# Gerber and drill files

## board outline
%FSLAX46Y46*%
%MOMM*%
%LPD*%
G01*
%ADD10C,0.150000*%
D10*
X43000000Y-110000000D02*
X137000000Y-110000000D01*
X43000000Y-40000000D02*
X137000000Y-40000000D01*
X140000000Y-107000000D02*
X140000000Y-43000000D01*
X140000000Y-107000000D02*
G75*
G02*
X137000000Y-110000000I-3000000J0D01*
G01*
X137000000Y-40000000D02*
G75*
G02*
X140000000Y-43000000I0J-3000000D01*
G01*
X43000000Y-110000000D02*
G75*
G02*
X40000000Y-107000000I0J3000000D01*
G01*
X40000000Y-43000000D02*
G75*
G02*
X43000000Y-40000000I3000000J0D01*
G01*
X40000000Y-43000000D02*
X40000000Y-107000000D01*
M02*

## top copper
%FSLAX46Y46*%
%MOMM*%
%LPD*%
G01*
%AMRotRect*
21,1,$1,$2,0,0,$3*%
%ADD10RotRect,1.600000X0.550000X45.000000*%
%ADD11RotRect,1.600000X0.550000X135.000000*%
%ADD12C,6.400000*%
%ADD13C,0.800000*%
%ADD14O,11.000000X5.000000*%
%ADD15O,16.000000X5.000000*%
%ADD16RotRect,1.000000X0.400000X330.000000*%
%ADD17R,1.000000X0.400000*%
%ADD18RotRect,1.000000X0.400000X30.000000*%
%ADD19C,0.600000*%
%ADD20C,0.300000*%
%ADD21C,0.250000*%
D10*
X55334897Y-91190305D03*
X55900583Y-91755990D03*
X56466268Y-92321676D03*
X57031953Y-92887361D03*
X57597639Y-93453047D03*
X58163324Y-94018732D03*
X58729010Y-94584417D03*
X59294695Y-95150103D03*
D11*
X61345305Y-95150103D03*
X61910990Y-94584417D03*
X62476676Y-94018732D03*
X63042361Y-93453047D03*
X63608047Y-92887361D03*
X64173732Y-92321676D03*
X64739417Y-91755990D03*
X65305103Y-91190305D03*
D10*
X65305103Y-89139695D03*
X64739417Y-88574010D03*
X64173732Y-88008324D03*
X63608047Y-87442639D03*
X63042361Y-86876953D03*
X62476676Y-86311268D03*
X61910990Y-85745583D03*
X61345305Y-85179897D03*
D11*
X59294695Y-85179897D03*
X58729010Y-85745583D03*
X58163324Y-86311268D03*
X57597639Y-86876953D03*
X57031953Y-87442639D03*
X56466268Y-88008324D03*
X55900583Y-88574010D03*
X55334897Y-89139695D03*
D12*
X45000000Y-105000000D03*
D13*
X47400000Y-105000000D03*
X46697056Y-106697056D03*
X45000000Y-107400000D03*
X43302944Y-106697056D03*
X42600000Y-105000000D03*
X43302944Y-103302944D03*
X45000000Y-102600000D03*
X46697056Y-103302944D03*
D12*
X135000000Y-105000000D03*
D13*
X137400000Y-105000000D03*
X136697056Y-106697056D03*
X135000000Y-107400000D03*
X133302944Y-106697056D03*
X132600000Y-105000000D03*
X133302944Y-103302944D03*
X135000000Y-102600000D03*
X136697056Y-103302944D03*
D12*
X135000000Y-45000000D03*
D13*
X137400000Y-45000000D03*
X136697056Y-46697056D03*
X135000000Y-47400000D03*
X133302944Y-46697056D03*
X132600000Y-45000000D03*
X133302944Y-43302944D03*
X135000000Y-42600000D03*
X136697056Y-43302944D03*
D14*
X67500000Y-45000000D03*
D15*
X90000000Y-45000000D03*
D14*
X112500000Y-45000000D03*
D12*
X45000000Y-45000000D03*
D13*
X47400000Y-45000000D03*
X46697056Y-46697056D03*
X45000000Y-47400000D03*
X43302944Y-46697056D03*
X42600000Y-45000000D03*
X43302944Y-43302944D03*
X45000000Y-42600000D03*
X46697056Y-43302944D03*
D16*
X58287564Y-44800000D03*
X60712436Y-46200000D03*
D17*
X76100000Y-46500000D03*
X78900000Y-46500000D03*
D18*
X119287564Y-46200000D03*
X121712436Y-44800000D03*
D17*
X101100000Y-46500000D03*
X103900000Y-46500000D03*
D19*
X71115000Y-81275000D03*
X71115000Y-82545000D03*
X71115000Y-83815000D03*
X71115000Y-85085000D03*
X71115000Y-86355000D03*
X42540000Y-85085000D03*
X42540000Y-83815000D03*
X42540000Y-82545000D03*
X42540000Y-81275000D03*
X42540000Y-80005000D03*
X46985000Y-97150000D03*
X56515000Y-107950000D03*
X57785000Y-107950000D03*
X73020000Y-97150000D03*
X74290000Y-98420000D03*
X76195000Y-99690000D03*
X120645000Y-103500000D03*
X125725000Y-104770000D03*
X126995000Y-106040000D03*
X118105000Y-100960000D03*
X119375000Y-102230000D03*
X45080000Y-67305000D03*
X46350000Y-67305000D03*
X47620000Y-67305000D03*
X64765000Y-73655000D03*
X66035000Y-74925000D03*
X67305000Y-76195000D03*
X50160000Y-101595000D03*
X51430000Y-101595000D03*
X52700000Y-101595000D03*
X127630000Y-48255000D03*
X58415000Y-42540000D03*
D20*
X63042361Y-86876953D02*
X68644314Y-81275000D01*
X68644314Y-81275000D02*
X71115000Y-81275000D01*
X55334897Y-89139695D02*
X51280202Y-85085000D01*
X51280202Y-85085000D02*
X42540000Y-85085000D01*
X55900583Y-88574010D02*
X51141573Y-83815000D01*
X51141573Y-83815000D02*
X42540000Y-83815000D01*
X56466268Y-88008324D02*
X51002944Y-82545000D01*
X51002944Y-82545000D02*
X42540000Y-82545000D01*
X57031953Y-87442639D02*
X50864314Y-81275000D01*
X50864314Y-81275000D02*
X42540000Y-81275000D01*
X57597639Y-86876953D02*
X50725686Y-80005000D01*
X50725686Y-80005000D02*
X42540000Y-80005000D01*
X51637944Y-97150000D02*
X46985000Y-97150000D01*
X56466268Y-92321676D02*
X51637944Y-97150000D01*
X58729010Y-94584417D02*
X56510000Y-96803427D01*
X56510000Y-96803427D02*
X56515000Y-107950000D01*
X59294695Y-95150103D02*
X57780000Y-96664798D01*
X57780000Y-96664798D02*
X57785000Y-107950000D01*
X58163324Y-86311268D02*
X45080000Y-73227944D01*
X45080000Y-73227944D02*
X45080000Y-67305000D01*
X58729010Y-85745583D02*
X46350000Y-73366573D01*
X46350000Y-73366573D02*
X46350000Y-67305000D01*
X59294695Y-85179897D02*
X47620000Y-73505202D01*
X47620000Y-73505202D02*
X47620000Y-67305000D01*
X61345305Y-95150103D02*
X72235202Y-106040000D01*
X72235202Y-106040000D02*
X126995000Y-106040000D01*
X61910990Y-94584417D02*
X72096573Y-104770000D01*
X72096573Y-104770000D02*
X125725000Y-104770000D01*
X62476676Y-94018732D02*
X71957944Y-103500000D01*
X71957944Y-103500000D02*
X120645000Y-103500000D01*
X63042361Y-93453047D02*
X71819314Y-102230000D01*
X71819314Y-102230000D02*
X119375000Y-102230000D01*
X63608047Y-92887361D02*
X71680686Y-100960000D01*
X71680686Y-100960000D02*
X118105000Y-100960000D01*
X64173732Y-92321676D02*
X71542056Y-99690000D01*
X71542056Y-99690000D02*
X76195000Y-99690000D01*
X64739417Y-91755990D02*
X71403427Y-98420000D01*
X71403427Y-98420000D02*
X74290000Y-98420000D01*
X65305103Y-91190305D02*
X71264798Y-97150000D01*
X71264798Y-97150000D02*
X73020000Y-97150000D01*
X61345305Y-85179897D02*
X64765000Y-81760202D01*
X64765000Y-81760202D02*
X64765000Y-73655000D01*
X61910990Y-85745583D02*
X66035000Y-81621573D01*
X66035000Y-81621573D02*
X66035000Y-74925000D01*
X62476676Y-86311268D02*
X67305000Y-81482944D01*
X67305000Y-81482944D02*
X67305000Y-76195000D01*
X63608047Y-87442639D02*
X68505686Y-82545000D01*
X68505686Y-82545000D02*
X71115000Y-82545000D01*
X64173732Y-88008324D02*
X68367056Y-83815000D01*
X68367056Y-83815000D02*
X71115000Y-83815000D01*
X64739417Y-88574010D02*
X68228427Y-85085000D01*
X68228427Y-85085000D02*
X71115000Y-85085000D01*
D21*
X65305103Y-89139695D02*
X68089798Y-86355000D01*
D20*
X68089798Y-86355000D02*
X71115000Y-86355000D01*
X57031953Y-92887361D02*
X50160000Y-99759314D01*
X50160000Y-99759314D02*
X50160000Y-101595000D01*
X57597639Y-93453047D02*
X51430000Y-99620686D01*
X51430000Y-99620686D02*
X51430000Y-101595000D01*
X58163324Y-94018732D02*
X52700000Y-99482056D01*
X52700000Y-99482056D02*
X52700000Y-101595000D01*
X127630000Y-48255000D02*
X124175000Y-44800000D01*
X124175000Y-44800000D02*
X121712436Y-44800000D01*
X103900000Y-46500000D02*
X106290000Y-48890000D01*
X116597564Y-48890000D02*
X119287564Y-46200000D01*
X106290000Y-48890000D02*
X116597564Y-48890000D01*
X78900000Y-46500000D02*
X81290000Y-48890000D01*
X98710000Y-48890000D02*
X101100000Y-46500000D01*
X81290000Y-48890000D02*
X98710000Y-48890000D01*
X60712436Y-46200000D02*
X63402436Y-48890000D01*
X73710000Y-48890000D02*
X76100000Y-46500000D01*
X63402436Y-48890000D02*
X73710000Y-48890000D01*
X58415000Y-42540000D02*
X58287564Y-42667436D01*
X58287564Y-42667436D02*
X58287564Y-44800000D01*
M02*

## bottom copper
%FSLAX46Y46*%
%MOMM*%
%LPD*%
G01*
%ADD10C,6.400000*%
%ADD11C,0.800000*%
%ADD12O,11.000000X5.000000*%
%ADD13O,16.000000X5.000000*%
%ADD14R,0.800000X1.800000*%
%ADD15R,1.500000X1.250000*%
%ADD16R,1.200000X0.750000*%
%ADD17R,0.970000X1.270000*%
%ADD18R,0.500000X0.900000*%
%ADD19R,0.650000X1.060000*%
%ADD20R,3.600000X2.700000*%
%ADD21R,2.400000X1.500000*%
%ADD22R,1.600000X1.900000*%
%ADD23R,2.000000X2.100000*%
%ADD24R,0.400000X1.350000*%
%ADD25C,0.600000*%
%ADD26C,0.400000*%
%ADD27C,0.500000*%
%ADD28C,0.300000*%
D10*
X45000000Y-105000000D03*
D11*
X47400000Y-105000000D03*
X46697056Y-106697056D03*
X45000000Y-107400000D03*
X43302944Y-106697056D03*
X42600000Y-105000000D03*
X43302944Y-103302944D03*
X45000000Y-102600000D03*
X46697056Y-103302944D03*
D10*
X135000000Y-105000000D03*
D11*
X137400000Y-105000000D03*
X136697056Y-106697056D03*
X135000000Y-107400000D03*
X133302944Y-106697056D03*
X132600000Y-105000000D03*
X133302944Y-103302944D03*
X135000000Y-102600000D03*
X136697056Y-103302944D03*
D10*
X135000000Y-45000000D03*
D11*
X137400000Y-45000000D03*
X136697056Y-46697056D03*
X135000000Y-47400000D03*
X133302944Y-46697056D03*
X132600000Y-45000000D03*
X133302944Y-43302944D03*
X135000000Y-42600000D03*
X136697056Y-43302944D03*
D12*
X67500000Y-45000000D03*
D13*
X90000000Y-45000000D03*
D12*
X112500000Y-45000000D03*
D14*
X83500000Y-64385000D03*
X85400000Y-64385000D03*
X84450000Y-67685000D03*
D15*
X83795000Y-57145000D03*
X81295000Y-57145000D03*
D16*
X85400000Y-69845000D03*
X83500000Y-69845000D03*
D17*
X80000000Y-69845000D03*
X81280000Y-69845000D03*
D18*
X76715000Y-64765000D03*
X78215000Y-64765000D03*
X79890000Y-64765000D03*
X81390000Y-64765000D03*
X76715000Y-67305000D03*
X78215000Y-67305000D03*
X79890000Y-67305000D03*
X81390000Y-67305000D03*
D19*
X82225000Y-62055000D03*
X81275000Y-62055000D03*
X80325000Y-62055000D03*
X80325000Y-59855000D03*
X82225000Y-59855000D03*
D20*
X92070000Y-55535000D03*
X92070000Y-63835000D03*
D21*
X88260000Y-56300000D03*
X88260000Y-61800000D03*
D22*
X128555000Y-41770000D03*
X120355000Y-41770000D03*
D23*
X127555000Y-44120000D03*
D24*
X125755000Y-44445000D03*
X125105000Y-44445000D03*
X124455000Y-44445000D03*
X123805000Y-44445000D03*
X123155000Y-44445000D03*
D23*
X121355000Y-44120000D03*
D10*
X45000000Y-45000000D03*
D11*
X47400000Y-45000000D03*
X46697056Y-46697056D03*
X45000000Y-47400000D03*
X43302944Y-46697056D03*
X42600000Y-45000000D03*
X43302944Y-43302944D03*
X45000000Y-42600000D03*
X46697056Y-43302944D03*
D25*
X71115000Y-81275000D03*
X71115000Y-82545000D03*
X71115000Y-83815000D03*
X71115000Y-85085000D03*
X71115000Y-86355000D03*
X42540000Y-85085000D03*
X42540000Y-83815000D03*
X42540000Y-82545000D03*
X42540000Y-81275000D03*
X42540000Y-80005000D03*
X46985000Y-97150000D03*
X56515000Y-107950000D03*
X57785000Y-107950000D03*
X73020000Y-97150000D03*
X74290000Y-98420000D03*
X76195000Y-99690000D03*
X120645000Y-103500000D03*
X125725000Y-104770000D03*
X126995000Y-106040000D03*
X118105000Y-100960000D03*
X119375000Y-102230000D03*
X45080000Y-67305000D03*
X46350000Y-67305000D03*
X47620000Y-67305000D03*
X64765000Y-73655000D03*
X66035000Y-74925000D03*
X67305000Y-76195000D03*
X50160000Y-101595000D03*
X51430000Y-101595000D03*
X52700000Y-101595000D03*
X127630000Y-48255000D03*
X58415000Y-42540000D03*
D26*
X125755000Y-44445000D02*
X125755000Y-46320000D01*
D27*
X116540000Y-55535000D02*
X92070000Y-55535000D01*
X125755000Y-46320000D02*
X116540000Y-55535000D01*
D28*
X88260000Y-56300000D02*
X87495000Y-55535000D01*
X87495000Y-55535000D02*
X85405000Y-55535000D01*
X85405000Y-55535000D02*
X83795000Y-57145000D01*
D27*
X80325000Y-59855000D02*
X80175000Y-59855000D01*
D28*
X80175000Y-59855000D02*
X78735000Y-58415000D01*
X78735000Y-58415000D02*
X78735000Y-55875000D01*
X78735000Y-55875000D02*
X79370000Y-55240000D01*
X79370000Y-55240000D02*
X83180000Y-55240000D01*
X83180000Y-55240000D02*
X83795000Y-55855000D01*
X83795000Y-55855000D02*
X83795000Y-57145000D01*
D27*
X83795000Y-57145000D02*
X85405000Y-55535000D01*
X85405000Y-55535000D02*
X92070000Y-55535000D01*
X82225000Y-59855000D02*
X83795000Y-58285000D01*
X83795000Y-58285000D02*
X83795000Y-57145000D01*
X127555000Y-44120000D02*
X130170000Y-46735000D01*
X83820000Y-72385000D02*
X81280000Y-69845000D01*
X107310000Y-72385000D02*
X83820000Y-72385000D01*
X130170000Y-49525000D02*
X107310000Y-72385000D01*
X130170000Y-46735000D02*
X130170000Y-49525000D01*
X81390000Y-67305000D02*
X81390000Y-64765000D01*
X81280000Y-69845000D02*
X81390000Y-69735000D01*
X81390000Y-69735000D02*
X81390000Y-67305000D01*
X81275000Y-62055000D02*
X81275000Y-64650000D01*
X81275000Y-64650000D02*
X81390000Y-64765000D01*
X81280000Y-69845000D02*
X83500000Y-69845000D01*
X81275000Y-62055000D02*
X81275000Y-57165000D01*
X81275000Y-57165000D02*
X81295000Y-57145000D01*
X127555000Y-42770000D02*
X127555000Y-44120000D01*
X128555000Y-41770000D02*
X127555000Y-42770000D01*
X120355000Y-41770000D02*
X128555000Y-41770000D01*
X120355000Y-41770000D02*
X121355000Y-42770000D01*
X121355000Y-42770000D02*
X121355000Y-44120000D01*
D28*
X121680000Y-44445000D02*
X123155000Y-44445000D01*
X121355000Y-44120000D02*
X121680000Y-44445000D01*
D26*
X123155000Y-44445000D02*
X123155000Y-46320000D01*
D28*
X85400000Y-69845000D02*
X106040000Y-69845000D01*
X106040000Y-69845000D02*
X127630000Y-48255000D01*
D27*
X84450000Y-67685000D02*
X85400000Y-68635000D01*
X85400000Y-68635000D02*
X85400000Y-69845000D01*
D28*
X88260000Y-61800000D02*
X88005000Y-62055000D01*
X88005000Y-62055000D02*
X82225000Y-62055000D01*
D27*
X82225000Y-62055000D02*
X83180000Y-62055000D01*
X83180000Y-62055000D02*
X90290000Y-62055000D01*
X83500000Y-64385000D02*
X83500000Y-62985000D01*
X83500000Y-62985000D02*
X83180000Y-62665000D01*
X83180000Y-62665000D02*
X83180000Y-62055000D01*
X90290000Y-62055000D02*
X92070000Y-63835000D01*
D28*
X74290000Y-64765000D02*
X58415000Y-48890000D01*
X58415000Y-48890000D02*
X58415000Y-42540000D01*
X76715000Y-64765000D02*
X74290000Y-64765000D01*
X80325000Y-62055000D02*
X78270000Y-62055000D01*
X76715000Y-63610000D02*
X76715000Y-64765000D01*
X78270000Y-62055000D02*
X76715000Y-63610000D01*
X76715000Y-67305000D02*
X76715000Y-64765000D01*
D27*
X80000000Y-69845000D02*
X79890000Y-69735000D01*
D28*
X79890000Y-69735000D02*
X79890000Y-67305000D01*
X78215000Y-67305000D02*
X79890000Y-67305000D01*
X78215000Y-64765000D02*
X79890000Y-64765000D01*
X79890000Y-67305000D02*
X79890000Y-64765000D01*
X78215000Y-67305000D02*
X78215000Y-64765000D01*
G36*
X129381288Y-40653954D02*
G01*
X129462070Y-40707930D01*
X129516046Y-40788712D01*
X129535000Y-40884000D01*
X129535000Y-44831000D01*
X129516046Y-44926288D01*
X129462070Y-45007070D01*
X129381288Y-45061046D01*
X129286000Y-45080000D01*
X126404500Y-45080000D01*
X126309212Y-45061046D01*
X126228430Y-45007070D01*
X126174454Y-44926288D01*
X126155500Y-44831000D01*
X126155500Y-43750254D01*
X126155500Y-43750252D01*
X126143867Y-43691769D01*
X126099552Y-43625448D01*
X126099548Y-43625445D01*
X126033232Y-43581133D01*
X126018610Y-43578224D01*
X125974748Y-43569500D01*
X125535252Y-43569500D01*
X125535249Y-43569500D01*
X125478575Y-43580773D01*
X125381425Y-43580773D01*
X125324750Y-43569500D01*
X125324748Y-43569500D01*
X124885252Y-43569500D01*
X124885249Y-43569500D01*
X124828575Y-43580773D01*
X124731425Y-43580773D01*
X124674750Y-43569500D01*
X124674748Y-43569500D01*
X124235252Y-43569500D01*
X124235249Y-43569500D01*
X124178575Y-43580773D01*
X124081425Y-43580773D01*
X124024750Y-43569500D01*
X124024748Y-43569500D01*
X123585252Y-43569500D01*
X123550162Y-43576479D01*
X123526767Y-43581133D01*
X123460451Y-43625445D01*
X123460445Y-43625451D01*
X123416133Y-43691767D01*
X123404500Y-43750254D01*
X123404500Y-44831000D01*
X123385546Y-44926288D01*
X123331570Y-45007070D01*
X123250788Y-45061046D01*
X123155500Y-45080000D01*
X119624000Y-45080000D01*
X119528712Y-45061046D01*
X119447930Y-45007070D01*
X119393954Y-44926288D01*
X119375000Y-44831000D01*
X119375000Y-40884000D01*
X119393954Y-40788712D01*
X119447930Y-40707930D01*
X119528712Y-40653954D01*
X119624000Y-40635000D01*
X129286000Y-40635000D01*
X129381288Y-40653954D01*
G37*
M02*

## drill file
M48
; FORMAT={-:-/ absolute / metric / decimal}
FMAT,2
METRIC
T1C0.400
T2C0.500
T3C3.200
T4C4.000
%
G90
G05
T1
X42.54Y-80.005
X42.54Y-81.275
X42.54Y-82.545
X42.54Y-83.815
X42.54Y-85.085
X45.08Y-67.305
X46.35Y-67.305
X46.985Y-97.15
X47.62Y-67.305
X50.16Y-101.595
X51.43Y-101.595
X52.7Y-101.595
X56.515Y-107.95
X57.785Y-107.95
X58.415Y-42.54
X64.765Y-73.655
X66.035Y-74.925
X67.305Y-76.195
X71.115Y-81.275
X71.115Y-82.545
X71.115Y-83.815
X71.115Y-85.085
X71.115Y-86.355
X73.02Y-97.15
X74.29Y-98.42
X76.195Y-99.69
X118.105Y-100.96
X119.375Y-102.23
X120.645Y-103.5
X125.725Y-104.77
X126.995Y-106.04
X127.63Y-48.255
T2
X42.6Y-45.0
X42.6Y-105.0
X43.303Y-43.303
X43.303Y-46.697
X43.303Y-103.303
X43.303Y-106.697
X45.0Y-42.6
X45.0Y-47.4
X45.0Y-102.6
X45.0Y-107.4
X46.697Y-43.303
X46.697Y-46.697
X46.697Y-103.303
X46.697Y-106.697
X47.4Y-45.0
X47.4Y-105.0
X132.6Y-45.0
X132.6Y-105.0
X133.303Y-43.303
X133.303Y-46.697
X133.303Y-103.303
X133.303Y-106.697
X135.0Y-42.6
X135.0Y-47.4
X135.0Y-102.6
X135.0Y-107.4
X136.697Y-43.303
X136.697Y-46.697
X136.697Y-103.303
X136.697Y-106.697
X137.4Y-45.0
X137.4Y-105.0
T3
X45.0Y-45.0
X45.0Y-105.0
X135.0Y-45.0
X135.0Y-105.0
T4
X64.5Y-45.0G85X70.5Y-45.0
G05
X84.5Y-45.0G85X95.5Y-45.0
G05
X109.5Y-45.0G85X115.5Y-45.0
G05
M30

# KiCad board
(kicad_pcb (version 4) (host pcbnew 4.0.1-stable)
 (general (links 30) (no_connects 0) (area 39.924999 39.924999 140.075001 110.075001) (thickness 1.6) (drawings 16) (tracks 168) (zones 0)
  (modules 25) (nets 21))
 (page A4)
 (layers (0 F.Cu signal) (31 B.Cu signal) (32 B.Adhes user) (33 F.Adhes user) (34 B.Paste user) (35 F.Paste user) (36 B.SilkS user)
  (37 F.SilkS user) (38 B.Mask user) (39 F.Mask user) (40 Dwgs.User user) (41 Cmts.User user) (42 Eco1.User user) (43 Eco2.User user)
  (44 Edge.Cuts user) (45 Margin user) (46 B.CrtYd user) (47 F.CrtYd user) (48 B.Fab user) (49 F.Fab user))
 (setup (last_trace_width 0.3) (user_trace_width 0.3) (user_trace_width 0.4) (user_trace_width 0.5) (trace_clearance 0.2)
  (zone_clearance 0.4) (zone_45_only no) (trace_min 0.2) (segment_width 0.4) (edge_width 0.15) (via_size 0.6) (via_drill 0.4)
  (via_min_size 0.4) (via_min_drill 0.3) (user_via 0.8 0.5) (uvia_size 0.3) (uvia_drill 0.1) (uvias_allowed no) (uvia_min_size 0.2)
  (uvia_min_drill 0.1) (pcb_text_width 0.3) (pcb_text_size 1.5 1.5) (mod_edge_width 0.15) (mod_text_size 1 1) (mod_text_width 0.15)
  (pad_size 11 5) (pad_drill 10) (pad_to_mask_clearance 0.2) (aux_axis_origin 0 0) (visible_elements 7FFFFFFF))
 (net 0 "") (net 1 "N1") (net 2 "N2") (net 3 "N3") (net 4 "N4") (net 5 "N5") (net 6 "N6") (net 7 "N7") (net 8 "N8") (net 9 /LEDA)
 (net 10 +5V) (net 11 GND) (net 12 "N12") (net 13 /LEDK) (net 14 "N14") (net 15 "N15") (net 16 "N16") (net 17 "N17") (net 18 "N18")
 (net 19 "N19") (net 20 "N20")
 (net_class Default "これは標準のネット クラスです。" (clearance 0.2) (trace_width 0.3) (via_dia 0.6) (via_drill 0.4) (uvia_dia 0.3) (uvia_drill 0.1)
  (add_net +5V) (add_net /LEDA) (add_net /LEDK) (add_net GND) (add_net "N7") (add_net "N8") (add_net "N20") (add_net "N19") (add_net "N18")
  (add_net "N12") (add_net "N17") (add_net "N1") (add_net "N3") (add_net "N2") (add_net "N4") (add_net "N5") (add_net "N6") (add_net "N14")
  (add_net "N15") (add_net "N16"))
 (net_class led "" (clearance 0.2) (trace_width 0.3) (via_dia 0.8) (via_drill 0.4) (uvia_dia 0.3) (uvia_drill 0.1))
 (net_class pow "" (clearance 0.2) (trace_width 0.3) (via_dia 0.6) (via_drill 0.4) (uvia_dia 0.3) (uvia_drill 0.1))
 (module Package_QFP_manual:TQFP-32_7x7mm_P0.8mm (layer F.Cu) (at 60.32 90.165 45)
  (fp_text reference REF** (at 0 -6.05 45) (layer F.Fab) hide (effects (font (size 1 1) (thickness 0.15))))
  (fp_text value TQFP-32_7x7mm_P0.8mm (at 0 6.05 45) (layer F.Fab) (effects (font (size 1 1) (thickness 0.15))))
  (pad 1 smd rect (at -4.25 -2.8 45) (size 1.6 0.55) (layers F.Cu F.Paste F.Mask))
  (pad 2 smd rect (at -4.25 -2 45) (size 1.6 0.55) (layers F.Cu F.Paste F.Mask))
  (pad 3 smd rect (at -4.25 -1.2 45) (size 1.6 0.55) (layers F.Cu F.Paste F.Mask))
  (pad 4 smd rect (at -4.25 -0.4 45) (size 1.6 0.55) (layers F.Cu F.Paste F.Mask))
  (pad 5 smd rect (at -4.25 0.4 45) (size 1.6 0.55) (layers F.Cu F.Paste F.Mask))
  (pad 6 smd rect (at -4.25 1.2 45) (size 1.6 0.55) (layers F.Cu F.Paste F.Mask))
  (pad 7 smd rect (at -4.25 2 45) (size 1.6 0.55) (layers F.Cu F.Paste F.Mask))
  (pad 8 smd rect (at -4.25 2.8 45) (size 1.6 0.55) (layers F.Cu F.Paste F.Mask))
  (pad 9 smd rect (at -2.8 4.25 135) (size 1.6 0.55) (layers F.Cu F.Paste F.Mask))
  (pad 10 smd rect (at -2 4.25 135) (size 1.6 0.55) (layers F.Cu F.Paste F.Mask))
  (pad 11 smd rect (at -1.2 4.25 135) (size 1.6 0.55) (layers F.Cu F.Paste F.Mask))
  (pad 12 smd rect (at -0.4 4.25 135) (size 1.6 0.55) (layers F.Cu F.Paste F.Mask))
  (pad 13 smd rect (at 0.4 4.25 135) (size 1.6 0.55) (layers F.Cu F.Paste F.Mask))
  (pad 14 smd rect (at 1.2 4.25 135) (size 1.6 0.55) (layers F.Cu F.Paste F.Mask))
  (pad 15 smd rect (at 2 4.25 135) (size 1.6 0.55) (layers F.Cu F.Paste F.Mask))
  (pad 16 smd rect (at 2.8 4.25 135) (size 1.6 0.55) (layers F.Cu F.Paste F.Mask))
  (pad 17 smd rect (at 4.25 2.8 45) (size 1.6 0.55) (layers F.Cu F.Paste F.Mask))
  (pad 18 smd rect (at 4.25 2 45) (size 1.6 0.55) (layers F.Cu F.Paste F.Mask))
  (pad 19 smd rect (at 4.25 1.2 45) (size 1.6 0.55) (layers F.Cu F.Paste F.Mask))
  (pad 20 smd rect (at 4.25 0.4 45) (size 1.6 0.55) (layers F.Cu F.Paste F.Mask))
  (pad 21 smd rect (at 4.25 -0.4 45) (size 1.6 0.55) (layers F.Cu F.Paste F.Mask))
  (pad 22 smd rect (at 4.25 -1.2 45) (size 1.6 0.55) (layers F.Cu F.Paste F.Mask))
  (pad 23 smd rect (at 4.25 -2 45) (size 1.6 0.55) (layers F.Cu F.Paste F.Mask))
  (pad 24 smd rect (at 4.25 -2.8 45) (size 1.6 0.55) (layers F.Cu F.Paste F.Mask))
  (pad 25 smd rect (at 2.8 -4.25 135) (size 1.6 0.55) (layers F.Cu F.Paste F.Mask))
  (pad 26 smd rect (at 2 -4.25 135) (size 1.6 0.55) (layers F.Cu F.Paste F.Mask))
  (pad 27 smd rect (at 1.2 -4.25 135) (size 1.6 0.55) (layers F.Cu F.Paste F.Mask))
  (pad 28 smd rect (at 0.4 -4.25 135) (size 1.6 0.55) (layers F.Cu F.Paste F.Mask))
  (pad 29 smd rect (at -0.4 -4.25 135) (size 1.6 0.55) (layers F.Cu F.Paste F.Mask))
  (pad 30 smd rect (at -1.2 -4.25 135) (size 1.6 0.55) (layers F.Cu F.Paste F.Mask))
  (pad 31 smd rect (at -2 -4.25 135) (size 1.6 0.55) (layers F.Cu F.Paste F.Mask))
  (pad 32 smd rect (at -2.8 -4.25 135) (size 1.6 0.55) (layers F.Cu F.Paste F.Mask)))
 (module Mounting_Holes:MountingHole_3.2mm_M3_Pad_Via (layer F.Cu) (at 45 105)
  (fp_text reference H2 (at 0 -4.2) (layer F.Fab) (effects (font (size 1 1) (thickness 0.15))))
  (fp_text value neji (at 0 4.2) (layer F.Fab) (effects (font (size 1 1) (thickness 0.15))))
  (pad 1 thru_hole circle (at 0 0) (size 6.4 6.4) (drill 3.2) (layers *.Cu *.Mask) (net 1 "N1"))
  (pad "" thru_hole circle (at 2.4 0) (size 0.8 0.8) (drill 0.5) (layers *.Cu *.Mask))
  (pad "" thru_hole circle (at 1.697056 1.697056) (size 0.8 0.8) (drill 0.5) (layers *.Cu *.Mask))
  (pad "" thru_hole circle (at 0 2.4) (size 0.8 0.8) (drill 0.5) (layers *.Cu *.Mask))
  (pad "" thru_hole circle (at -1.697056 1.697056) (size 0.8 0.8) (drill 0.5) (layers *.Cu *.Mask))
  (pad "" thru_hole circle (at -2.4 0) (size 0.8 0.8) (drill 0.5) (layers *.Cu *.Mask))
  (pad "" thru_hole circle (at -1.697056 -1.697056) (size 0.8 0.8) (drill 0.5) (layers *.Cu *.Mask))
  (pad "" thru_hole circle (at 0 -2.4) (size 0.8 0.8) (drill 0.5) (layers *.Cu *.Mask))
  (pad "" thru_hole circle (at 1.697056 -1.697056) (size 0.8 0.8) (drill 0.5) (layers *.Cu *.Mask)))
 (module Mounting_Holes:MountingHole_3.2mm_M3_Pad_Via (layer F.Cu) (at 135 105)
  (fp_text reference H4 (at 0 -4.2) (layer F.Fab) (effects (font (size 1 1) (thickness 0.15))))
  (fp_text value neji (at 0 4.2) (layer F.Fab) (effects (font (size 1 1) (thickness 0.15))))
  (pad 1 thru_hole circle (at 0 0) (size 6.4 6.4) (drill 3.2) (layers *.Cu *.Mask) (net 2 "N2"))
  (pad "" thru_hole circle (at 2.4 0) (size 0.8 0.8) (drill 0.5) (layers *.Cu *.Mask))
  (pad "" thru_hole circle (at 1.697056 1.697056) (size 0.8 0.8) (drill 0.5) (layers *.Cu *.Mask))
  (pad "" thru_hole circle (at 0 2.4) (size 0.8 0.8) (drill 0.5) (layers *.Cu *.Mask))
  (pad "" thru_hole circle (at -1.697056 1.697056) (size 0.8 0.8) (drill 0.5) (layers *.Cu *.Mask))
  (pad "" thru_hole circle (at -2.4 0) (size 0.8 0.8) (drill 0.5) (layers *.Cu *.Mask))
  (pad "" thru_hole circle (at -1.697056 -1.697056) (size 0.8 0.8) (drill 0.5) (layers *.Cu *.Mask))
  (pad "" thru_hole circle (at 0 -2.4) (size 0.8 0.8) (drill 0.5) (layers *.Cu *.Mask))
  (pad "" thru_hole circle (at 1.697056 -1.697056) (size 0.8 0.8) (drill 0.5) (layers *.Cu *.Mask)))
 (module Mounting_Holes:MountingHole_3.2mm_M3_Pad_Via (layer F.Cu) (at 135 45)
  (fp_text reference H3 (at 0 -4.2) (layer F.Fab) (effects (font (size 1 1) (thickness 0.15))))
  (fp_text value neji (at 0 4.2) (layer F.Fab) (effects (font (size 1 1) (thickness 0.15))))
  (pad 1 thru_hole circle (at 0 0) (size 6.4 6.4) (drill 3.2) (layers *.Cu *.Mask) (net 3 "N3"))
  (pad "" thru_hole circle (at 2.4 0) (size 0.8 0.8) (drill 0.5) (layers *.Cu *.Mask))
  (pad "" thru_hole circle (at 1.697056 1.697056) (size 0.8 0.8) (drill 0.5) (layers *.Cu *.Mask))
  (pad "" thru_hole circle (at 0 2.4) (size 0.8 0.8) (drill 0.5) (layers *.Cu *.Mask))
  (pad "" thru_hole circle (at -1.697056 1.697056) (size 0.8 0.8) (drill 0.5) (layers *.Cu *.Mask))
  (pad "" thru_hole circle (at -2.4 0) (size 0.8 0.8) (drill 0.5) (layers *.Cu *.Mask))
  (pad "" thru_hole circle (at -1.697056 -1.697056) (size 0.8 0.8) (drill 0.5) (layers *.Cu *.Mask))
  (pad "" thru_hole circle (at 0 -2.4) (size 0.8 0.8) (drill 0.5) (layers *.Cu *.Mask))
  (pad "" thru_hole circle (at 1.697056 -1.697056) (size 0.8 0.8) (drill 0.5) (layers *.Cu *.Mask)))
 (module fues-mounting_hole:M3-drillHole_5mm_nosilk (layer F.Cu) (at 67.5 45)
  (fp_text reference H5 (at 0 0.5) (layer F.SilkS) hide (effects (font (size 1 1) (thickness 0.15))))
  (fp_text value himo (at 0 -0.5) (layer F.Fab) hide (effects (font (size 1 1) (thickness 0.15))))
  (pad 1 thru_hole oval (at 0 0) (size 11 5) (drill oval 10 4) (layers *.Cu *.Mask) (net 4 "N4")))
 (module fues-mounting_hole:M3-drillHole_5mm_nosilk (layer F.Cu) (at 90 45)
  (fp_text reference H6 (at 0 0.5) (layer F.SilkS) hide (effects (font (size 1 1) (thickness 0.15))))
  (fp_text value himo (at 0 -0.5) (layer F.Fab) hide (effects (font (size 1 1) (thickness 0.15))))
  (pad 1 thru_hole oval (at 0 0) (size 16 5) (drill oval 15 4) (layers *.Cu *.Mask) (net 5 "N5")))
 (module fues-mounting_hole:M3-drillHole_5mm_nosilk (layer F.Cu) (at 112.5 45)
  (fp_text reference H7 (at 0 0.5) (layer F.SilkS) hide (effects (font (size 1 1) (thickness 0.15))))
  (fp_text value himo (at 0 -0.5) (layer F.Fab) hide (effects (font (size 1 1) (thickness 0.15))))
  (pad 1 thru_hole oval (at 0 0) (size 11 5) (drill oval 10 4) (layers *.Cu *.Mask) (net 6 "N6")))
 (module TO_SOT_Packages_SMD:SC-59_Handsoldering (layer B.Cu) (at 84.45 66.035 270)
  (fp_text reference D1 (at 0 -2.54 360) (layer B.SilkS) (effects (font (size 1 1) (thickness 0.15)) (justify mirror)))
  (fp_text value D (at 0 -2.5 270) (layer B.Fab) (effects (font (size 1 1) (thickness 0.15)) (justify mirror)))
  (pad 1 smd rect (at -1.65 0.95 270) (size 1.8 0.8) (layers B.Cu B.Paste B.Mask) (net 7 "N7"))
  (pad 2 smd rect (at -1.65 -0.95 270) (size 1.8 0.8) (layers B.Cu B.Paste B.Mask) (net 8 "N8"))
  (pad 3 smd rect (at 1.65 0 270) (size 1.8 0.8) (layers B.Cu B.Paste B.Mask) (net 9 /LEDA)))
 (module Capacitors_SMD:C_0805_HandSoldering (layer B.Cu) (at 82.545 57.145 180)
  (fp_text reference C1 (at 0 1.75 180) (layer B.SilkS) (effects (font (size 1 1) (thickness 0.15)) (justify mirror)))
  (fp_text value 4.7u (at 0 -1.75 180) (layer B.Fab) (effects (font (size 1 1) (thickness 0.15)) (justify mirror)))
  (pad 1 smd rect (at -1.25 0 180) (size 1.5 1.25) (layers B.Cu B.Paste B.Mask) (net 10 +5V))
  (pad 2 smd rect (at 1.25 0 180) (size 1.5 1.25) (layers B.Cu B.Paste B.Mask) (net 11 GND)))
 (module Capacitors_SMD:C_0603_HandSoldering (layer B.Cu) (at 84.45 69.845 180)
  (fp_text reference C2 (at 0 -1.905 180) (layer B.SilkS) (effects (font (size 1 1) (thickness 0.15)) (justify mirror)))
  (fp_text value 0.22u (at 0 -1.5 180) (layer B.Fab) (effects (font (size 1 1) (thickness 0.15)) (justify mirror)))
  (pad 1 smd rect (at -0.95 0 180) (size 1.2 0.75) (layers B.Cu B.Paste B.Mask) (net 9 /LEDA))
  (pad 2 smd rect (at 0.95 0 180) (size 1.2 0.75) (layers B.Cu B.Paste B.Mask) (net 11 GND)))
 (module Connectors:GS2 (layer B.Cu) (at 80.64 69.845 270)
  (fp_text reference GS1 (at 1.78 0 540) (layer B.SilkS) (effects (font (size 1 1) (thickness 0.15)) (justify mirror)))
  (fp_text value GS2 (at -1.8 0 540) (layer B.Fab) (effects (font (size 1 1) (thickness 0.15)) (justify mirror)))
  (pad 1 smd rect (at 0 0.64 270) (size 1.27 0.97) (layers B.Cu B.Paste B.Mask) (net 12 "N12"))
  (pad 2 smd rect (at 0 -0.64 270) (size 1.27 0.97) (layers B.Cu B.Paste B.Mask) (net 11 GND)))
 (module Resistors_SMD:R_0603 (layer B.Cu) (at 77.465 64.765)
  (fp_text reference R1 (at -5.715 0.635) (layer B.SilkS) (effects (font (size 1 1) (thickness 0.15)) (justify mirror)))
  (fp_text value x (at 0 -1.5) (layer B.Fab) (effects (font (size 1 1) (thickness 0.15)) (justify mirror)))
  (pad 1 smd rect (at -0.75 0) (size 0.5 0.9) (layers B.Cu B.Paste B.Mask) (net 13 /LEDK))
  (pad 2 smd rect (at 0.75 0) (size 0.5 0.9) (layers B.Cu B.Paste B.Mask) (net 12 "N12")))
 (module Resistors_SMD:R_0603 (layer B.Cu) (at 80.64 64.765)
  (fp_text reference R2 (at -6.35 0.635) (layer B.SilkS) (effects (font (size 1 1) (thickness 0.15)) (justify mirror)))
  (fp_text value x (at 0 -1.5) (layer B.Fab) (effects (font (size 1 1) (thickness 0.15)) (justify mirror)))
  (pad 1 smd rect (at -0.75 0) (size 0.5 0.9) (layers B.Cu B.Paste B.Mask) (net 12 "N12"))
  (pad 2 smd rect (at 0.75 0) (size 0.5 0.9) (layers B.Cu B.Paste B.Mask) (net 11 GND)))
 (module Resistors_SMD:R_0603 (layer B.Cu) (at 77.465 67.305)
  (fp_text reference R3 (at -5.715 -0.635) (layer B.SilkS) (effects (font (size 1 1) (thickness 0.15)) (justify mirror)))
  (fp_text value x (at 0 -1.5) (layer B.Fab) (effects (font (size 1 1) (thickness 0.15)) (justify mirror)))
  (pad 1 smd rect (at -0.75 0) (size 0.5 0.9) (layers B.Cu B.Paste B.Mask) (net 13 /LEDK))
  (pad 2 smd rect (at 0.75 0) (size 0.5 0.9) (layers B.Cu B.Paste B.Mask) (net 12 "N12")))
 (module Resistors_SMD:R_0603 (layer B.Cu) (at 80.64 67.305)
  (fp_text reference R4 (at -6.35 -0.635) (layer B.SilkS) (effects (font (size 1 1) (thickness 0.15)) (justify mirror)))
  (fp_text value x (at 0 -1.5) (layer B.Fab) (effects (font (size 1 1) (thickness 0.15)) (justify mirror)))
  (pad 1 smd rect (at -0.75 0) (size 0.5 0.9) (layers B.Cu B.Paste B.Mask) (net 12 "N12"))
  (pad 2 smd rect (at 0.75 0) (size 0.5 0.9) (layers B.Cu B.Paste B.Mask) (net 11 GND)))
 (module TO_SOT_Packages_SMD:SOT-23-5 (layer B.Cu) (at 81.275 60.955 90)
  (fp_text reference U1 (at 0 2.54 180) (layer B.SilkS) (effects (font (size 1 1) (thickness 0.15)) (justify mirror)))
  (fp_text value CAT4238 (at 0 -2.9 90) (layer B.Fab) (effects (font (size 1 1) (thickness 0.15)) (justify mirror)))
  (pad 1 smd rect (at -1.1 0.95 90) (size 1.06 0.65) (layers B.Cu B.Paste B.Mask) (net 7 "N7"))
  (pad 2 smd rect (at -1.1 0 90) (size 1.06 0.65) (layers B.Cu B.Paste B.Mask) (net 11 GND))
  (pad 3 smd rect (at -1.1 -0.95 90) (size 1.06 0.65) (layers B.Cu B.Paste B.Mask) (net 13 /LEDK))
  (pad 4 smd rect (at 1.1 -0.95 90) (size 1.06 0.65) (layers B.Cu B.Paste B.Mask) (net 10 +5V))
  (pad 5 smd rect (at 1.1 0.95 90) (size 1.06 0.65) (layers B.Cu B.Paste B.Mask) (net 10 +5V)))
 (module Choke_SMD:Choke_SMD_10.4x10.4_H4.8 (layer B.Cu) (at 92.07 59.685 270)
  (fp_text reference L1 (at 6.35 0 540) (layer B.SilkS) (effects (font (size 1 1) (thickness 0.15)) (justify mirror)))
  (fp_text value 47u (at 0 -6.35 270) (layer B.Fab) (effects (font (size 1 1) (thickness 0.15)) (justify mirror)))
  (pad 1 smd rect (at -4.15 0 270) (size 2.7 3.6) (layers B.Cu B.Paste B.Mask) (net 10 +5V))
  (pad 2 smd rect (at 4.15 0 270) (size 2.7 3.6) (layers B.Cu B.Paste B.Mask) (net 7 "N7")))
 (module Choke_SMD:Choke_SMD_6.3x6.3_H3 (layer B.Cu) (at 88.26 59.05 270)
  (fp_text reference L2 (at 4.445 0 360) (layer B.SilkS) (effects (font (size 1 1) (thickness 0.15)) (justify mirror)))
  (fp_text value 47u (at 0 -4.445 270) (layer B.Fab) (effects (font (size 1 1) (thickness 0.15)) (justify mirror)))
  (pad 1 smd rect (at -2.75 0 270) (size 1.5 2.4) (layers B.Cu B.Paste B.Mask) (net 10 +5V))
  (pad 2 smd rect (at 2.75 0 270) (size 1.5 2.4) (layers B.Cu B.Paste B.Mask) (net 7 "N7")))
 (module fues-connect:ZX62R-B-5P (layer B.Cu) (at 124.455 44.445 180)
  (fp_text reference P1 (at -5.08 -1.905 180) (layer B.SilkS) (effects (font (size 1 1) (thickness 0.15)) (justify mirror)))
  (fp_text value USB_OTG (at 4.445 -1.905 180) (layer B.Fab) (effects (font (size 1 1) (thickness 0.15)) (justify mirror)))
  (pad 6 smd rect (at -4.1 2.675 180) (size 1.6 1.9) (layers B.Cu B.Paste B.Mask) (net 11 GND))
  (pad 6 smd rect (at 4.1 2.675 180) (size 1.6 1.9) (layers B.Cu B.Paste B.Mask) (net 11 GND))
  (pad 6 smd rect (at -3.1 0.325 180) (size 2 2.1) (layers B.Cu B.Paste B.Mask) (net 11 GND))
  (pad 1 smd rect (at -1.3 0 180) (size 0.4 1.35) (layers B.Cu B.Paste B.Mask) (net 10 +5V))
  (pad 2 smd rect (at -0.65 0 180) (size 0.4 1.35) (layers B.Cu B.Paste B.Mask) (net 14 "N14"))
  (pad 3 smd rect (at 0 0 180) (size 0.4 1.35) (layers B.Cu B.Paste B.Mask) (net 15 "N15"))
  (pad 4 smd rect (at 0.65 0 180) (size 0.4 1.35) (layers B.Cu B.Paste B.Mask) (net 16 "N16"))
  (pad 5 smd rect (at 1.3 0 180) (size 0.4 1.35) (layers B.Cu B.Paste B.Mask) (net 11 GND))
  (pad 6 smd rect (at 3.1 0.325 180) (size 2 2.1) (layers B.Cu B.Paste B.Mask) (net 11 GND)))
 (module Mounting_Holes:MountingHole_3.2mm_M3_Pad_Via (layer F.Cu) (at 45 45)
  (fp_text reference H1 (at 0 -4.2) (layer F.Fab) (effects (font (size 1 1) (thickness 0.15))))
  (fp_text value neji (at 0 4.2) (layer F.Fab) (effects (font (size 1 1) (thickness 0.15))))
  (pad 1 thru_hole circle (at 0 0) (size 6.4 6.4) (drill 3.2) (layers *.Cu *.Mask) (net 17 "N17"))
  (pad "" thru_hole circle (at 2.4 0) (size 0.8 0.8) (drill 0.5) (layers *.Cu *.Mask))
  (pad "" thru_hole circle (at 1.697056 1.697056) (size 0.8 0.8) (drill 0.5) (layers *.Cu *.Mask))
  (pad "" thru_hole circle (at 0 2.4) (size 0.8 0.8) (drill 0.5) (layers *.Cu *.Mask))
  (pad "" thru_hole circle (at -1.697056 1.697056) (size 0.8 0.8) (drill 0.5) (layers *.Cu *.Mask))
  (pad "" thru_hole circle (at -2.4 0) (size 0.8 0.8) (drill 0.5) (layers *.Cu *.Mask))
  (pad "" thru_hole circle (at -1.697056 -1.697056) (size 0.8 0.8) (drill 0.5) (layers *.Cu *.Mask))
  (pad "" thru_hole circle (at 0 -2.4) (size 0.8 0.8) (drill 0.5) (layers *.Cu *.Mask))
  (pad "" thru_hole circle (at 1.697056 -1.697056) (size 0.8 0.8) (drill 0.5) (layers *.Cu *.Mask)))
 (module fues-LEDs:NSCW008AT (layer F.Cu) (at 59.5 45.5 330)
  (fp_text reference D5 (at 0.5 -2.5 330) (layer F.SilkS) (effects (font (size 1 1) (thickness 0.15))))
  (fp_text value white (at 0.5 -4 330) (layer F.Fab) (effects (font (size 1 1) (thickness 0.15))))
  (pad 1 smd rect (at -1.4 0 330) (size 1 0.4) (layers F.Cu F.Paste F.Mask) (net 13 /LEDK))
  (pad 2 smd rect (at 1.4 0 330) (size 1 0.4) (layers F.Cu F.Paste F.Mask) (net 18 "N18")))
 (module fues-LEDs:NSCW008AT (layer F.Cu) (at 77.5 46.5)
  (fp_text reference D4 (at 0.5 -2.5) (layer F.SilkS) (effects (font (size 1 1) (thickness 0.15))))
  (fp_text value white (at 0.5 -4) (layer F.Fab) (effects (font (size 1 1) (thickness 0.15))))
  (pad 1 smd rect (at -1.4 0) (size 1 0.4) (layers F.Cu F.Paste F.Mask) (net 18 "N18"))
  (pad 2 smd rect (at 1.4 0) (size 1 0.4) (layers F.Cu F.Paste F.Mask) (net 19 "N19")))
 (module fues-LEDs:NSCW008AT (layer F.Cu) (at 120.5 45.5 30)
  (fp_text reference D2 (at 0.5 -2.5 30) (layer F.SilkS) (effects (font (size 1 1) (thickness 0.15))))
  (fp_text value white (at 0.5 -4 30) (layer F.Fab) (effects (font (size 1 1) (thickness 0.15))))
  (pad 1 smd rect (at -1.4 0 30) (size 1 0.4) (layers F.Cu F.Paste F.Mask) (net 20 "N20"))
  (pad 2 smd rect (at 1.4 0 30) (size 1 0.4) (layers F.Cu F.Paste F.Mask) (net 9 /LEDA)))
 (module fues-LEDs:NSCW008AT (layer F.Cu) (at 102.5 46.5)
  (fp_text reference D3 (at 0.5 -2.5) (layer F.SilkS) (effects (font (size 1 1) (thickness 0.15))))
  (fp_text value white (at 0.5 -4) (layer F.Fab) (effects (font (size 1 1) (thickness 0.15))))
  (pad 1 smd rect (at -1.4 0) (size 1 0.4) (layers F.Cu F.Paste F.Mask) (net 19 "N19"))
  (pad 2 smd rect (at 1.4 0) (size 1 0.4) (layers F.Cu F.Paste F.Mask) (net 20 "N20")))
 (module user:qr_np (layer B.Cu) (at 133.35 76.2 180)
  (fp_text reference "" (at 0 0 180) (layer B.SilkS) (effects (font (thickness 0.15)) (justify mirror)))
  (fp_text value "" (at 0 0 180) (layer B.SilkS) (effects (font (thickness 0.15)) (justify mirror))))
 (gr_line (start 43 110) (end 137 110) (angle 90) (layer Edge.Cuts) (width 0.15))
 (gr_line (start 43 40) (end 137 40) (angle 90) (layer Edge.Cuts) (width 0.15))
 (gr_line (start 140 107) (end 140 43) (angle 90) (layer Edge.Cuts) (width 0.15))
 (gr_arc (start 137 107) (end 140 107) (angle 90) (layer Edge.Cuts) (width 0.15))
 (gr_arc (start 137 43) (end 137 40) (angle 90) (layer Edge.Cuts) (width 0.15))
 (gr_arc (start 43 107) (end 43 110) (angle 90) (layer Edge.Cuts) (width 0.15))
 (gr_arc (start 43 43) (end 40 43) (angle 90) (layer Edge.Cuts) (width 0.15))
 (gr_line (start 40 43) (end 40 107) (angle 90) (layer Edge.Cuts) (width 0.15))
 (via (at 71.115 81.275) (size 0.6) (drill 0.4) (layers F.Cu B.Cu) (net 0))
 (via (at 71.115 82.545) (size 0.6) (drill 0.4) (layers F.Cu B.Cu) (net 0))
 (via (at 71.115 83.815) (size 0.6) (drill 0.4) (layers F.Cu B.Cu) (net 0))
 (via (at 71.115 85.085) (size 0.6) (drill 0.4) (layers F.Cu B.Cu) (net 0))
 (via (at 71.115 86.355) (size 0.6) (drill 0.4) (layers F.Cu B.Cu) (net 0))
 (segment (start 63.042361 86.876953) (end 68.644314 81.275) (width 0.3) (layer F.Cu) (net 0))
 (segment (start 68.644314 81.275) (end 71.115 81.275) (width 0.3) (layer F.Cu) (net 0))
 (segment (start 55.334897 89.139695) (end 51.280202 85.085) (width 0.3) (layer F.Cu) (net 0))
 (via (at 42.54 85.085) (size 0.6) (drill 0.4) (layers F.Cu B.Cu) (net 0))
 (segment (start 51.280202 85.085) (end 42.54 85.085) (width 0.3) (layer F.Cu) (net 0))
 (segment (start 55.900583 88.57401) (end 51.141573 83.815) (width 0.3) (layer F.Cu) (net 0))
 (via (at 42.54 83.815) (size 0.6) (drill 0.4) (layers F.Cu B.Cu) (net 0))
 (segment (start 51.141573 83.815) (end 42.54 83.815) (width 0.3) (layer F.Cu) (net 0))
 (segment (start 56.466268 88.008324) (end 51.002944 82.545) (width 0.3) (layer F.Cu) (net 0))
 (via (at 42.54 82.545) (size 0.6) (drill 0.4) (layers F.Cu B.Cu) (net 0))
 (segment (start 51.002944 82.545) (end 42.54 82.545) (width 0.3) (layer F.Cu) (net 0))
 (segment (start 57.031953 87.442639) (end 50.864314 81.275) (width 0.3) (layer F.Cu) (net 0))
 (via (at 42.54 81.275) (size 0.6) (drill 0.4) (layers F.Cu B.Cu) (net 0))
 (segment (start 50.864314 81.275) (end 42.54 81.275) (width 0.3) (layer F.Cu) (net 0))
 (segment (start 57.597639 86.876953) (end 50.725686 80.005) (width 0.3) (layer F.Cu) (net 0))
 (via (at 42.54 80.005) (size 0.6) (drill 0.4) (layers F.Cu B.Cu) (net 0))
 (segment (start 50.725686 80.005) (end 42.54 80.005) (width 0.3) (layer F.Cu) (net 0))
 (via (at 46.985 97.15) (size 0.6) (drill 0.4) (layers F.Cu B.Cu) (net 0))
 (segment (start 51.637944 97.15) (end 46.985 97.15) (width 0.3) (layer F.Cu) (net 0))
 (segment (start 56.466268 92.321676) (end 51.637944 97.15) (width 0.3) (layer F.Cu) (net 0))
 (via (at 56.515 107.95) (size 0.6) (drill 0.4) (layers F.Cu B.Cu) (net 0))
 (via (at 57.785 107.95) (size 0.6) (drill 0.4) (layers F.Cu B.Cu) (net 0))
 (via (at 73.02 97.15) (size 0.6) (drill 0.4) (layers F.Cu B.Cu) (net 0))
 (via (at 74.29 98.42) (size 0.6) (drill 0.4) (layers F.Cu B.Cu) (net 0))
 (via (at 76.195 99.69) (size 0.6) (drill 0.4) (layers F.Cu B.Cu) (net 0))
 (via (at 120.645 103.5) (size 0.6) (drill 0.4) (layers F.Cu B.Cu) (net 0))
 (via (at 125.725 104.77) (size 0.6) (drill 0.4) (layers F.Cu B.Cu) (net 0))
 (via (at 126.995 106.04) (size 0.6) (drill 0.4) (layers F.Cu B.Cu) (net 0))
 (via (at 118.105 100.96) (size 0.6) (drill 0.4) (layers F.Cu B.Cu) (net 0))
 (via (at 119.375 102.23) (size 0.6) (drill 0.4) (layers F.Cu B.Cu) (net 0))
 (segment (start 58.72901 94.584417) (end 56.51 96.803427) (width 0.3) (layer F.Cu) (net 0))
 (segment (start 56.51 96.803427) (end 56.515 107.95) (width 0.3) (layer F.Cu) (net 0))
 (segment (start 59.294695 95.150103) (end 57.78 96.664798) (width 0.3) (layer F.Cu) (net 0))
 (segment (start 57.78 96.664798) (end 57.785 107.95) (width 0.3) (layer F.Cu) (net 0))
 (via (at 45.08 67.305) (size 0.6) (drill 0.4) (layers F.Cu B.Cu) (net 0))
 (via (at 46.35 67.305) (size 0.6) (drill 0.4) (layers F.Cu B.Cu) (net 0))
 (via (at 47.62 67.305) (size 0.6) (drill 0.4) (layers F.Cu B.Cu) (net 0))
 (via (at 64.765 73.655) (size 0.6) (drill 0.4) (layers F.Cu B.Cu) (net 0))
 (via (at 66.035 74.925) (size 0.6) (drill 0.4) (layers F.Cu B.Cu) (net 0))
 (segment (start 58.163324 86.311268) (end 45.08 73.227944) (width 0.3) (layer F.Cu) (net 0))
 (segment (start 45.08 73.227944) (end 45.08 67.305) (width 0.3) (layer F.Cu) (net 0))
 (segment (start 58.72901 85.745583) (end 46.35 73.366573) (width 0.3) (layer F.Cu) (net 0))
 (segment (start 46.35 73.366573) (end 46.35 67.305) (width 0.3) (layer F.Cu) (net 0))
 (segment (start 59.294695 85.179897) (end 47.62 73.505202) (width 0.3) (layer F.Cu) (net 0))
 (segment (start 47.62 73.505202) (end 47.62 67.305) (width 0.3) (layer F.Cu) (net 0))
 (segment (start 61.345305 95.150103) (end 72.235202 106.04) (width 0.3) (layer F.Cu) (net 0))
 (segment (start 72.235202 106.04) (end 126.995 106.04) (width 0.3) (layer F.Cu) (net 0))
 (segment (start 61.91099 94.584417) (end 72.096573 104.77) (width 0.3) (layer F.Cu) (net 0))
 (segment (start 72.096573 104.77) (end 125.725 104.77) (width 0.3) (layer F.Cu) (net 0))
 (segment (start 62.476676 94.018732) (end 71.957944 103.5) (width 0.3) (layer F.Cu) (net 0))
 (segment (start 71.957944 103.5) (end 120.645 103.5) (width 0.3) (layer F.Cu) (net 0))
 (segment (start 63.042361 93.453047) (end 71.819314 102.23) (width 0.3) (layer F.Cu) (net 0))
 (segment (start 71.819314 102.23) (end 119.375 102.23) (width 0.3) (layer F.Cu) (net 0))
 (segment (start 63.608047 92.887361) (end 71.680686 100.96) (width 0.3) (layer F.Cu) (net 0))
 (segment (start 71.680686 100.96) (end 118.105 100.96) (width 0.3) (layer F.Cu) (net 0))
 (segment (start 64.173732 92.321676) (end 71.542056 99.69) (width 0.3) (layer F.Cu) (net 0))
 (segment (start 71.542056 99.69) (end 76.195 99.69) (width 0.3) (layer F.Cu) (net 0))
 (segment (start 64.739417 91.75599) (end 71.403427 98.42) (width 0.3) (layer F.Cu) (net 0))
 (segment (start 71.403427 98.42) (end 74.29 98.42) (width 0.3) (layer F.Cu) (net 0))
 (segment (start 65.305103 91.190305) (end 71.264798 97.15) (width 0.3) (layer F.Cu) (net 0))
 (segment (start 71.264798 97.15) (end 73.02 97.15) (width 0.3) (layer F.Cu) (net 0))
 (segment (start 61.345305 85.179897) (end 64.765 81.760202) (width 0.3) (layer F.Cu) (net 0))
 (segment (start 64.765 81.760202) (end 64.765 73.655) (width 0.3) (layer F.Cu) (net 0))
 (segment (start 61.91099 85.745583) (end 66.035 81.621573) (width 0.3) (layer F.Cu) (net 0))
 (segment (start 66.035 81.621573) (end 66.035 74.925) (width 0.3) (layer F.Cu) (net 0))
 (segment (start 62.476676 86.311268) (end 67.305 81.482944) (width 0.3) (layer F.Cu) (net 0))
 (segment (start 67.305 81.482944) (end 67.305 76.195) (width 0.3) (layer F.Cu) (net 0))
 (via (at 67.305 76.195) (size 0.6) (drill 0.4) (layers F.Cu B.Cu) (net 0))
 (segment (start 63.608047 87.442639) (end 68.505686 82.545) (width 0.3) (layer F.Cu) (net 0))
 (segment (start 68.505686 82.545) (end 71.115 82.545) (width 0.3) (layer F.Cu) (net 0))
 (segment (start 64.173732 88.008324) (end 68.367056 83.815) (width 0.3) (layer F.Cu) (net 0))
 (segment (start 68.367056 83.815) (end 71.115 83.815) (width 0.3) (layer F.Cu) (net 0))
 (segment (start 64.739417 88.57401) (end 68.228427 85.085) (width 0.3) (layer F.Cu) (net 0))
 (segment (start 68.228427 85.085) (end 71.115 85.085) (width 0.3) (layer F.Cu) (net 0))
 (segment (start 65.305103 89.139695) (end 68.089798 86.355) (width 0.25) (layer F.Cu) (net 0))
 (segment (start 68.089798 86.355) (end 71.115 86.355) (width 0.3) (layer F.Cu) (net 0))
 (via (at 50.16 101.595) (size 0.6) (drill 0.4) (layers F.Cu B.Cu) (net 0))
 (via (at 51.43 101.595) (size 0.6) (drill 0.4) (layers F.Cu B.Cu) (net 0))
 (via (at 52.7 101.595) (size 0.6) (drill 0.4) (layers F.Cu B.Cu) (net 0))
 (segment (start 57.031953 92.887361) (end 50.16 99.759314) (width 0.3) (layer F.Cu) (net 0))
 (segment (start 50.16 99.759314) (end 50.16 101.595) (width 0.3) (layer F.Cu) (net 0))
 (segment (start 57.597639 93.453047) (end 51.43 99.620686) (width 0.3) (layer F.Cu) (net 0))
 (segment (start 51.43 99.620686) (end 51.43 101.595) (width 0.3) (layer F.Cu) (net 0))
 (segment (start 58.163324 94.018732) (end 52.7 99.482056) (width 0.3) (layer F.Cu) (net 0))
 (segment (start 52.7 99.482056) (end 52.7 101.595) (width 0.3) (layer F.Cu) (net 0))
 (segment (start 125.755 44.445) (end 125.755 46.32) (width 0.4) (layer B.Cu) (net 10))
 (segment (start 116.54 55.535) (end 92.07 55.535) (width 0.5) (layer B.Cu) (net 10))
 (segment (start 125.755 46.32) (end 116.54 55.535) (width 0.5) (layer B.Cu) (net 10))
 (segment (start 88.26 56.3) (end 87.495 55.535) (width 0.3) (layer B.Cu) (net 10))
 (segment (start 87.495 55.535) (end 85.405 55.535) (width 0.3) (layer B.Cu) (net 10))
 (segment (start 85.405 55.535) (end 83.795 57.145) (width 0.3) (layer B.Cu) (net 10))
 (segment (start 80.325 59.855) (end 80.175 59.855) (width 0.5) (layer B.Cu) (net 10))
 (segment (start 80.175 59.855) (end 78.735 58.415) (width 0.3) (layer B.Cu) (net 10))
 (segment (start 78.735 58.415) (end 78.735 55.875) (width 0.3) (layer B.Cu) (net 10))
 (segment (start 78.735 55.875) (end 79.37 55.24) (width 0.3) (layer B.Cu) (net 10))
 (segment (start 79.37 55.24) (end 83.18 55.24) (width 0.3) (layer B.Cu) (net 10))
 (segment (start 83.18 55.24) (end 83.795 55.855) (width 0.3) (layer B.Cu) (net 10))
 (segment (start 83.795 55.855) (end 83.795 57.145) (width 0.3) (layer B.Cu) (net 10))
 (segment (start 83.795 57.145) (end 85.405 55.535) (width 0.5) (layer B.Cu) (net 10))
 (segment (start 85.405 55.535) (end 92.07 55.535) (width 0.5) (layer B.Cu) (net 10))
 (segment (start 82.225 59.855) (end 83.795 58.285) (width 0.5) (layer B.Cu) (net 10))
 (segment (start 83.795 58.285) (end 83.795 57.145) (width 0.5) (layer B.Cu) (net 10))
 (segment (start 127.555 44.12) (end 130.17 46.735) (width 0.5) (layer B.Cu) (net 11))
 (segment (start 83.82 72.385) (end 81.28 69.845) (width 0.5) (layer B.Cu) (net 11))
 (segment (start 107.31 72.385) (end 83.82 72.385) (width 0.5) (layer B.Cu) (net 11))
 (segment (start 130.17 49.525) (end 107.31 72.385) (width 0.5) (layer B.Cu) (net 11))
 (segment (start 130.17 46.735) (end 130.17 49.525) (width 0.5) (layer B.Cu) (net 11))
 (segment (start 81.39 67.305) (end 81.39 64.765) (width 0.5) (layer B.Cu) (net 11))
 (segment (start 81.28 69.845) (end 81.39 69.735) (width 0.5) (layer B.Cu) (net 11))
 (segment (start 81.39 69.735) (end 81.39 67.305) (width 0.5) (layer B.Cu) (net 11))
 (segment (start 81.275 62.055) (end 81.275 64.65) (width 0.5) (layer B.Cu) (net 11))
 (segment (start 81.275 64.65) (end 81.39 64.765) (width 0.5) (layer B.Cu) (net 11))
 (segment (start 81.28 69.845) (end 83.5 69.845) (width 0.5) (layer B.Cu) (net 11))
 (segment (start 81.275 62.055) (end 81.275 57.165) (width 0.5) (layer B.Cu) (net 11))
 (segment (start 81.275 57.165) (end 81.295 57.145) (width 0.5) (layer B.Cu) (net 11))
 (segment (start 127.555 42.77) (end 127.555 44.12) (width 0.5) (layer B.Cu) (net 11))
 (segment (start 128.555 41.77) (end 127.555 42.77) (width 0.5) (layer B.Cu) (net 11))
 (segment (start 120.355 41.77) (end 128.555 41.77) (width 0.5) (layer B.Cu) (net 11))
 (segment (start 120.355 41.77) (end 121.355 42.77) (width 0.5) (layer B.Cu) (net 11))
 (segment (start 121.355 42.77) (end 121.355 44.12) (width 0.5) (layer B.Cu) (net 11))
 (segment (start 121.68 44.445) (end 123.155 44.445) (width 0.3) (layer B.Cu) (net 11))
 (segment (start 121.355 44.12) (end 121.68 44.445) (width 0.3) (layer B.Cu) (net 11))
 (segment (start 123.155 44.445) (end 123.155 46.32) (width 0.4) (layer B.Cu) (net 11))
 (segment (start 127.63 48.255) (end 124.175 44.8) (width 0.3) (layer F.Cu) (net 9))
 (segment (start 85.4 69.845) (end 106.04 69.845) (width 0.3) (layer B.Cu) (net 9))
 (via (at 127.63 48.255) (size 0.6) (drill 0.4) (layers F.Cu B.Cu) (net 9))
 (segment (start 106.04 69.845) (end 127.63 48.255) (width 0.3) (layer B.Cu) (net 9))
 (segment (start 124.175 44.8) (end 121.712436 44.8) (width 0.3) (layer F.Cu) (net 9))
 (segment (start 84.45 67.685) (end 85.4 68.635) (width 0.5) (layer B.Cu) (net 9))
 (segment (start 85.4 68.635) (end 85.4 69.845) (width 0.5) (layer B.Cu) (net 9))
 (segment (start 88.26 61.8) (end 88.005 62.055) (width 0.3) (layer B.Cu) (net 7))
 (segment (start 88.005 62.055) (end 82.225 62.055) (width 0.3) (layer B.Cu) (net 7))
 (segment (start 82.225 62.055) (end 83.18 62.055) (width 0.5) (layer B.Cu) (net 7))
 (segment (start 83.18 62.055) (end 90.29 62.055) (width 0.5) (layer B.Cu) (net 7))
 (segment (start 83.5 64.385) (end 83.5 62.985) (width 0.5) (layer B.Cu) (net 7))
 (segment (start 83.5 62.985) (end 83.18 62.665) (width 0.5) (layer B.Cu) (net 7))
 (segment (start 83.18 62.665) (end 83.18 62.055) (width 0.5) (layer B.Cu) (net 7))
 (segment (start 90.29 62.055) (end 92.07 63.835) (width 0.5) (layer B.Cu) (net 7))
 (segment (start 103.9 46.5) (end 106.29 48.89) (width 0.3) (layer F.Cu) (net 20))
 (segment (start 116.597564 48.89) (end 119.287564 46.2) (width 0.3) (layer F.Cu) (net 20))
 (segment (start 106.29 48.89) (end 116.597564 48.89) (width 0.3) (layer F.Cu) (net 20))
 (segment (start 78.9 46.5) (end 81.29 48.89) (width 0.3) (layer F.Cu) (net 19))
 (segment (start 98.71 48.89) (end 101.1 46.5) (width 0.3) (layer F.Cu) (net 19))
 (segment (start 81.29 48.89) (end 98.71 48.89) (width 0.3) (layer F.Cu) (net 19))
 (segment (start 60.712436 46.2) (end 63.402436 48.89) (width 0.3) (layer F.Cu) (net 18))
 (segment (start 73.71 48.89) (end 76.1 46.5) (width 0.3) (layer F.Cu) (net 18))
 (segment (start 63.402436 48.89) (end 73.71 48.89) (width 0.3) (layer F.Cu) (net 18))
 (segment (start 58.415 42.54) (end 58.287564 42.667436) (width 0.3) (layer F.Cu) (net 13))
 (segment (start 74.29 64.765) (end 58.415 48.89) (width 0.3) (layer B.Cu) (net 13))
 (segment (start 58.415 48.89) (end 58.415 42.54) (width 0.3) (layer B.Cu) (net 13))
 (via (at 58.415 42.54) (size 0.6) (drill 0.4) (layers F.Cu B.Cu) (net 13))
 (segment (start 76.715 64.765) (end 74.29 64.765) (width 0.3) (layer B.Cu) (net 13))
 (segment (start 58.287564 42.667436) (end 58.287564 44.8) (width 0.3) (layer F.Cu) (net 13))
 (segment (start 80.325 62.055) (end 78.27 62.055) (width 0.3) (layer B.Cu) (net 13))
 (segment (start 76.715 63.61) (end 76.715 64.765) (width 0.3) (layer B.Cu) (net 13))
 (segment (start 78.27 62.055) (end 76.715 63.61) (width 0.3) (layer B.Cu) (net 13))
 (segment (start 76.715 67.305) (end 76.715 64.765) (width 0.3) (layer B.Cu) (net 13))
 (segment (start 80 69.845) (end 79.89 69.735) (width 0.5) (layer B.Cu) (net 12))
 (segment (start 79.89 69.735) (end 79.89 67.305) (width 0.3) (layer B.Cu) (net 12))
 (segment (start 78.215 67.305) (end 79.89 67.305) (width 0.3) (layer B.Cu) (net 12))
 (segment (start 78.215 64.765) (end 79.89 64.765) (width 0.3) (layer B.Cu) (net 12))
 (segment (start 79.89 67.305) (end 79.89 64.765) (width 0.3) (layer B.Cu) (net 12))
 (segment (start 78.215 67.305) (end 78.215 64.765) (width 0.3) (layer B.Cu) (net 12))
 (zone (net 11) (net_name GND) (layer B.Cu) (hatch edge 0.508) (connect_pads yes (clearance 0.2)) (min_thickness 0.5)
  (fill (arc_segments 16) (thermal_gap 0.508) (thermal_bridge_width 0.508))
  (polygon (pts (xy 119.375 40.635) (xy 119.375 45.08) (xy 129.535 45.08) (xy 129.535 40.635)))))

